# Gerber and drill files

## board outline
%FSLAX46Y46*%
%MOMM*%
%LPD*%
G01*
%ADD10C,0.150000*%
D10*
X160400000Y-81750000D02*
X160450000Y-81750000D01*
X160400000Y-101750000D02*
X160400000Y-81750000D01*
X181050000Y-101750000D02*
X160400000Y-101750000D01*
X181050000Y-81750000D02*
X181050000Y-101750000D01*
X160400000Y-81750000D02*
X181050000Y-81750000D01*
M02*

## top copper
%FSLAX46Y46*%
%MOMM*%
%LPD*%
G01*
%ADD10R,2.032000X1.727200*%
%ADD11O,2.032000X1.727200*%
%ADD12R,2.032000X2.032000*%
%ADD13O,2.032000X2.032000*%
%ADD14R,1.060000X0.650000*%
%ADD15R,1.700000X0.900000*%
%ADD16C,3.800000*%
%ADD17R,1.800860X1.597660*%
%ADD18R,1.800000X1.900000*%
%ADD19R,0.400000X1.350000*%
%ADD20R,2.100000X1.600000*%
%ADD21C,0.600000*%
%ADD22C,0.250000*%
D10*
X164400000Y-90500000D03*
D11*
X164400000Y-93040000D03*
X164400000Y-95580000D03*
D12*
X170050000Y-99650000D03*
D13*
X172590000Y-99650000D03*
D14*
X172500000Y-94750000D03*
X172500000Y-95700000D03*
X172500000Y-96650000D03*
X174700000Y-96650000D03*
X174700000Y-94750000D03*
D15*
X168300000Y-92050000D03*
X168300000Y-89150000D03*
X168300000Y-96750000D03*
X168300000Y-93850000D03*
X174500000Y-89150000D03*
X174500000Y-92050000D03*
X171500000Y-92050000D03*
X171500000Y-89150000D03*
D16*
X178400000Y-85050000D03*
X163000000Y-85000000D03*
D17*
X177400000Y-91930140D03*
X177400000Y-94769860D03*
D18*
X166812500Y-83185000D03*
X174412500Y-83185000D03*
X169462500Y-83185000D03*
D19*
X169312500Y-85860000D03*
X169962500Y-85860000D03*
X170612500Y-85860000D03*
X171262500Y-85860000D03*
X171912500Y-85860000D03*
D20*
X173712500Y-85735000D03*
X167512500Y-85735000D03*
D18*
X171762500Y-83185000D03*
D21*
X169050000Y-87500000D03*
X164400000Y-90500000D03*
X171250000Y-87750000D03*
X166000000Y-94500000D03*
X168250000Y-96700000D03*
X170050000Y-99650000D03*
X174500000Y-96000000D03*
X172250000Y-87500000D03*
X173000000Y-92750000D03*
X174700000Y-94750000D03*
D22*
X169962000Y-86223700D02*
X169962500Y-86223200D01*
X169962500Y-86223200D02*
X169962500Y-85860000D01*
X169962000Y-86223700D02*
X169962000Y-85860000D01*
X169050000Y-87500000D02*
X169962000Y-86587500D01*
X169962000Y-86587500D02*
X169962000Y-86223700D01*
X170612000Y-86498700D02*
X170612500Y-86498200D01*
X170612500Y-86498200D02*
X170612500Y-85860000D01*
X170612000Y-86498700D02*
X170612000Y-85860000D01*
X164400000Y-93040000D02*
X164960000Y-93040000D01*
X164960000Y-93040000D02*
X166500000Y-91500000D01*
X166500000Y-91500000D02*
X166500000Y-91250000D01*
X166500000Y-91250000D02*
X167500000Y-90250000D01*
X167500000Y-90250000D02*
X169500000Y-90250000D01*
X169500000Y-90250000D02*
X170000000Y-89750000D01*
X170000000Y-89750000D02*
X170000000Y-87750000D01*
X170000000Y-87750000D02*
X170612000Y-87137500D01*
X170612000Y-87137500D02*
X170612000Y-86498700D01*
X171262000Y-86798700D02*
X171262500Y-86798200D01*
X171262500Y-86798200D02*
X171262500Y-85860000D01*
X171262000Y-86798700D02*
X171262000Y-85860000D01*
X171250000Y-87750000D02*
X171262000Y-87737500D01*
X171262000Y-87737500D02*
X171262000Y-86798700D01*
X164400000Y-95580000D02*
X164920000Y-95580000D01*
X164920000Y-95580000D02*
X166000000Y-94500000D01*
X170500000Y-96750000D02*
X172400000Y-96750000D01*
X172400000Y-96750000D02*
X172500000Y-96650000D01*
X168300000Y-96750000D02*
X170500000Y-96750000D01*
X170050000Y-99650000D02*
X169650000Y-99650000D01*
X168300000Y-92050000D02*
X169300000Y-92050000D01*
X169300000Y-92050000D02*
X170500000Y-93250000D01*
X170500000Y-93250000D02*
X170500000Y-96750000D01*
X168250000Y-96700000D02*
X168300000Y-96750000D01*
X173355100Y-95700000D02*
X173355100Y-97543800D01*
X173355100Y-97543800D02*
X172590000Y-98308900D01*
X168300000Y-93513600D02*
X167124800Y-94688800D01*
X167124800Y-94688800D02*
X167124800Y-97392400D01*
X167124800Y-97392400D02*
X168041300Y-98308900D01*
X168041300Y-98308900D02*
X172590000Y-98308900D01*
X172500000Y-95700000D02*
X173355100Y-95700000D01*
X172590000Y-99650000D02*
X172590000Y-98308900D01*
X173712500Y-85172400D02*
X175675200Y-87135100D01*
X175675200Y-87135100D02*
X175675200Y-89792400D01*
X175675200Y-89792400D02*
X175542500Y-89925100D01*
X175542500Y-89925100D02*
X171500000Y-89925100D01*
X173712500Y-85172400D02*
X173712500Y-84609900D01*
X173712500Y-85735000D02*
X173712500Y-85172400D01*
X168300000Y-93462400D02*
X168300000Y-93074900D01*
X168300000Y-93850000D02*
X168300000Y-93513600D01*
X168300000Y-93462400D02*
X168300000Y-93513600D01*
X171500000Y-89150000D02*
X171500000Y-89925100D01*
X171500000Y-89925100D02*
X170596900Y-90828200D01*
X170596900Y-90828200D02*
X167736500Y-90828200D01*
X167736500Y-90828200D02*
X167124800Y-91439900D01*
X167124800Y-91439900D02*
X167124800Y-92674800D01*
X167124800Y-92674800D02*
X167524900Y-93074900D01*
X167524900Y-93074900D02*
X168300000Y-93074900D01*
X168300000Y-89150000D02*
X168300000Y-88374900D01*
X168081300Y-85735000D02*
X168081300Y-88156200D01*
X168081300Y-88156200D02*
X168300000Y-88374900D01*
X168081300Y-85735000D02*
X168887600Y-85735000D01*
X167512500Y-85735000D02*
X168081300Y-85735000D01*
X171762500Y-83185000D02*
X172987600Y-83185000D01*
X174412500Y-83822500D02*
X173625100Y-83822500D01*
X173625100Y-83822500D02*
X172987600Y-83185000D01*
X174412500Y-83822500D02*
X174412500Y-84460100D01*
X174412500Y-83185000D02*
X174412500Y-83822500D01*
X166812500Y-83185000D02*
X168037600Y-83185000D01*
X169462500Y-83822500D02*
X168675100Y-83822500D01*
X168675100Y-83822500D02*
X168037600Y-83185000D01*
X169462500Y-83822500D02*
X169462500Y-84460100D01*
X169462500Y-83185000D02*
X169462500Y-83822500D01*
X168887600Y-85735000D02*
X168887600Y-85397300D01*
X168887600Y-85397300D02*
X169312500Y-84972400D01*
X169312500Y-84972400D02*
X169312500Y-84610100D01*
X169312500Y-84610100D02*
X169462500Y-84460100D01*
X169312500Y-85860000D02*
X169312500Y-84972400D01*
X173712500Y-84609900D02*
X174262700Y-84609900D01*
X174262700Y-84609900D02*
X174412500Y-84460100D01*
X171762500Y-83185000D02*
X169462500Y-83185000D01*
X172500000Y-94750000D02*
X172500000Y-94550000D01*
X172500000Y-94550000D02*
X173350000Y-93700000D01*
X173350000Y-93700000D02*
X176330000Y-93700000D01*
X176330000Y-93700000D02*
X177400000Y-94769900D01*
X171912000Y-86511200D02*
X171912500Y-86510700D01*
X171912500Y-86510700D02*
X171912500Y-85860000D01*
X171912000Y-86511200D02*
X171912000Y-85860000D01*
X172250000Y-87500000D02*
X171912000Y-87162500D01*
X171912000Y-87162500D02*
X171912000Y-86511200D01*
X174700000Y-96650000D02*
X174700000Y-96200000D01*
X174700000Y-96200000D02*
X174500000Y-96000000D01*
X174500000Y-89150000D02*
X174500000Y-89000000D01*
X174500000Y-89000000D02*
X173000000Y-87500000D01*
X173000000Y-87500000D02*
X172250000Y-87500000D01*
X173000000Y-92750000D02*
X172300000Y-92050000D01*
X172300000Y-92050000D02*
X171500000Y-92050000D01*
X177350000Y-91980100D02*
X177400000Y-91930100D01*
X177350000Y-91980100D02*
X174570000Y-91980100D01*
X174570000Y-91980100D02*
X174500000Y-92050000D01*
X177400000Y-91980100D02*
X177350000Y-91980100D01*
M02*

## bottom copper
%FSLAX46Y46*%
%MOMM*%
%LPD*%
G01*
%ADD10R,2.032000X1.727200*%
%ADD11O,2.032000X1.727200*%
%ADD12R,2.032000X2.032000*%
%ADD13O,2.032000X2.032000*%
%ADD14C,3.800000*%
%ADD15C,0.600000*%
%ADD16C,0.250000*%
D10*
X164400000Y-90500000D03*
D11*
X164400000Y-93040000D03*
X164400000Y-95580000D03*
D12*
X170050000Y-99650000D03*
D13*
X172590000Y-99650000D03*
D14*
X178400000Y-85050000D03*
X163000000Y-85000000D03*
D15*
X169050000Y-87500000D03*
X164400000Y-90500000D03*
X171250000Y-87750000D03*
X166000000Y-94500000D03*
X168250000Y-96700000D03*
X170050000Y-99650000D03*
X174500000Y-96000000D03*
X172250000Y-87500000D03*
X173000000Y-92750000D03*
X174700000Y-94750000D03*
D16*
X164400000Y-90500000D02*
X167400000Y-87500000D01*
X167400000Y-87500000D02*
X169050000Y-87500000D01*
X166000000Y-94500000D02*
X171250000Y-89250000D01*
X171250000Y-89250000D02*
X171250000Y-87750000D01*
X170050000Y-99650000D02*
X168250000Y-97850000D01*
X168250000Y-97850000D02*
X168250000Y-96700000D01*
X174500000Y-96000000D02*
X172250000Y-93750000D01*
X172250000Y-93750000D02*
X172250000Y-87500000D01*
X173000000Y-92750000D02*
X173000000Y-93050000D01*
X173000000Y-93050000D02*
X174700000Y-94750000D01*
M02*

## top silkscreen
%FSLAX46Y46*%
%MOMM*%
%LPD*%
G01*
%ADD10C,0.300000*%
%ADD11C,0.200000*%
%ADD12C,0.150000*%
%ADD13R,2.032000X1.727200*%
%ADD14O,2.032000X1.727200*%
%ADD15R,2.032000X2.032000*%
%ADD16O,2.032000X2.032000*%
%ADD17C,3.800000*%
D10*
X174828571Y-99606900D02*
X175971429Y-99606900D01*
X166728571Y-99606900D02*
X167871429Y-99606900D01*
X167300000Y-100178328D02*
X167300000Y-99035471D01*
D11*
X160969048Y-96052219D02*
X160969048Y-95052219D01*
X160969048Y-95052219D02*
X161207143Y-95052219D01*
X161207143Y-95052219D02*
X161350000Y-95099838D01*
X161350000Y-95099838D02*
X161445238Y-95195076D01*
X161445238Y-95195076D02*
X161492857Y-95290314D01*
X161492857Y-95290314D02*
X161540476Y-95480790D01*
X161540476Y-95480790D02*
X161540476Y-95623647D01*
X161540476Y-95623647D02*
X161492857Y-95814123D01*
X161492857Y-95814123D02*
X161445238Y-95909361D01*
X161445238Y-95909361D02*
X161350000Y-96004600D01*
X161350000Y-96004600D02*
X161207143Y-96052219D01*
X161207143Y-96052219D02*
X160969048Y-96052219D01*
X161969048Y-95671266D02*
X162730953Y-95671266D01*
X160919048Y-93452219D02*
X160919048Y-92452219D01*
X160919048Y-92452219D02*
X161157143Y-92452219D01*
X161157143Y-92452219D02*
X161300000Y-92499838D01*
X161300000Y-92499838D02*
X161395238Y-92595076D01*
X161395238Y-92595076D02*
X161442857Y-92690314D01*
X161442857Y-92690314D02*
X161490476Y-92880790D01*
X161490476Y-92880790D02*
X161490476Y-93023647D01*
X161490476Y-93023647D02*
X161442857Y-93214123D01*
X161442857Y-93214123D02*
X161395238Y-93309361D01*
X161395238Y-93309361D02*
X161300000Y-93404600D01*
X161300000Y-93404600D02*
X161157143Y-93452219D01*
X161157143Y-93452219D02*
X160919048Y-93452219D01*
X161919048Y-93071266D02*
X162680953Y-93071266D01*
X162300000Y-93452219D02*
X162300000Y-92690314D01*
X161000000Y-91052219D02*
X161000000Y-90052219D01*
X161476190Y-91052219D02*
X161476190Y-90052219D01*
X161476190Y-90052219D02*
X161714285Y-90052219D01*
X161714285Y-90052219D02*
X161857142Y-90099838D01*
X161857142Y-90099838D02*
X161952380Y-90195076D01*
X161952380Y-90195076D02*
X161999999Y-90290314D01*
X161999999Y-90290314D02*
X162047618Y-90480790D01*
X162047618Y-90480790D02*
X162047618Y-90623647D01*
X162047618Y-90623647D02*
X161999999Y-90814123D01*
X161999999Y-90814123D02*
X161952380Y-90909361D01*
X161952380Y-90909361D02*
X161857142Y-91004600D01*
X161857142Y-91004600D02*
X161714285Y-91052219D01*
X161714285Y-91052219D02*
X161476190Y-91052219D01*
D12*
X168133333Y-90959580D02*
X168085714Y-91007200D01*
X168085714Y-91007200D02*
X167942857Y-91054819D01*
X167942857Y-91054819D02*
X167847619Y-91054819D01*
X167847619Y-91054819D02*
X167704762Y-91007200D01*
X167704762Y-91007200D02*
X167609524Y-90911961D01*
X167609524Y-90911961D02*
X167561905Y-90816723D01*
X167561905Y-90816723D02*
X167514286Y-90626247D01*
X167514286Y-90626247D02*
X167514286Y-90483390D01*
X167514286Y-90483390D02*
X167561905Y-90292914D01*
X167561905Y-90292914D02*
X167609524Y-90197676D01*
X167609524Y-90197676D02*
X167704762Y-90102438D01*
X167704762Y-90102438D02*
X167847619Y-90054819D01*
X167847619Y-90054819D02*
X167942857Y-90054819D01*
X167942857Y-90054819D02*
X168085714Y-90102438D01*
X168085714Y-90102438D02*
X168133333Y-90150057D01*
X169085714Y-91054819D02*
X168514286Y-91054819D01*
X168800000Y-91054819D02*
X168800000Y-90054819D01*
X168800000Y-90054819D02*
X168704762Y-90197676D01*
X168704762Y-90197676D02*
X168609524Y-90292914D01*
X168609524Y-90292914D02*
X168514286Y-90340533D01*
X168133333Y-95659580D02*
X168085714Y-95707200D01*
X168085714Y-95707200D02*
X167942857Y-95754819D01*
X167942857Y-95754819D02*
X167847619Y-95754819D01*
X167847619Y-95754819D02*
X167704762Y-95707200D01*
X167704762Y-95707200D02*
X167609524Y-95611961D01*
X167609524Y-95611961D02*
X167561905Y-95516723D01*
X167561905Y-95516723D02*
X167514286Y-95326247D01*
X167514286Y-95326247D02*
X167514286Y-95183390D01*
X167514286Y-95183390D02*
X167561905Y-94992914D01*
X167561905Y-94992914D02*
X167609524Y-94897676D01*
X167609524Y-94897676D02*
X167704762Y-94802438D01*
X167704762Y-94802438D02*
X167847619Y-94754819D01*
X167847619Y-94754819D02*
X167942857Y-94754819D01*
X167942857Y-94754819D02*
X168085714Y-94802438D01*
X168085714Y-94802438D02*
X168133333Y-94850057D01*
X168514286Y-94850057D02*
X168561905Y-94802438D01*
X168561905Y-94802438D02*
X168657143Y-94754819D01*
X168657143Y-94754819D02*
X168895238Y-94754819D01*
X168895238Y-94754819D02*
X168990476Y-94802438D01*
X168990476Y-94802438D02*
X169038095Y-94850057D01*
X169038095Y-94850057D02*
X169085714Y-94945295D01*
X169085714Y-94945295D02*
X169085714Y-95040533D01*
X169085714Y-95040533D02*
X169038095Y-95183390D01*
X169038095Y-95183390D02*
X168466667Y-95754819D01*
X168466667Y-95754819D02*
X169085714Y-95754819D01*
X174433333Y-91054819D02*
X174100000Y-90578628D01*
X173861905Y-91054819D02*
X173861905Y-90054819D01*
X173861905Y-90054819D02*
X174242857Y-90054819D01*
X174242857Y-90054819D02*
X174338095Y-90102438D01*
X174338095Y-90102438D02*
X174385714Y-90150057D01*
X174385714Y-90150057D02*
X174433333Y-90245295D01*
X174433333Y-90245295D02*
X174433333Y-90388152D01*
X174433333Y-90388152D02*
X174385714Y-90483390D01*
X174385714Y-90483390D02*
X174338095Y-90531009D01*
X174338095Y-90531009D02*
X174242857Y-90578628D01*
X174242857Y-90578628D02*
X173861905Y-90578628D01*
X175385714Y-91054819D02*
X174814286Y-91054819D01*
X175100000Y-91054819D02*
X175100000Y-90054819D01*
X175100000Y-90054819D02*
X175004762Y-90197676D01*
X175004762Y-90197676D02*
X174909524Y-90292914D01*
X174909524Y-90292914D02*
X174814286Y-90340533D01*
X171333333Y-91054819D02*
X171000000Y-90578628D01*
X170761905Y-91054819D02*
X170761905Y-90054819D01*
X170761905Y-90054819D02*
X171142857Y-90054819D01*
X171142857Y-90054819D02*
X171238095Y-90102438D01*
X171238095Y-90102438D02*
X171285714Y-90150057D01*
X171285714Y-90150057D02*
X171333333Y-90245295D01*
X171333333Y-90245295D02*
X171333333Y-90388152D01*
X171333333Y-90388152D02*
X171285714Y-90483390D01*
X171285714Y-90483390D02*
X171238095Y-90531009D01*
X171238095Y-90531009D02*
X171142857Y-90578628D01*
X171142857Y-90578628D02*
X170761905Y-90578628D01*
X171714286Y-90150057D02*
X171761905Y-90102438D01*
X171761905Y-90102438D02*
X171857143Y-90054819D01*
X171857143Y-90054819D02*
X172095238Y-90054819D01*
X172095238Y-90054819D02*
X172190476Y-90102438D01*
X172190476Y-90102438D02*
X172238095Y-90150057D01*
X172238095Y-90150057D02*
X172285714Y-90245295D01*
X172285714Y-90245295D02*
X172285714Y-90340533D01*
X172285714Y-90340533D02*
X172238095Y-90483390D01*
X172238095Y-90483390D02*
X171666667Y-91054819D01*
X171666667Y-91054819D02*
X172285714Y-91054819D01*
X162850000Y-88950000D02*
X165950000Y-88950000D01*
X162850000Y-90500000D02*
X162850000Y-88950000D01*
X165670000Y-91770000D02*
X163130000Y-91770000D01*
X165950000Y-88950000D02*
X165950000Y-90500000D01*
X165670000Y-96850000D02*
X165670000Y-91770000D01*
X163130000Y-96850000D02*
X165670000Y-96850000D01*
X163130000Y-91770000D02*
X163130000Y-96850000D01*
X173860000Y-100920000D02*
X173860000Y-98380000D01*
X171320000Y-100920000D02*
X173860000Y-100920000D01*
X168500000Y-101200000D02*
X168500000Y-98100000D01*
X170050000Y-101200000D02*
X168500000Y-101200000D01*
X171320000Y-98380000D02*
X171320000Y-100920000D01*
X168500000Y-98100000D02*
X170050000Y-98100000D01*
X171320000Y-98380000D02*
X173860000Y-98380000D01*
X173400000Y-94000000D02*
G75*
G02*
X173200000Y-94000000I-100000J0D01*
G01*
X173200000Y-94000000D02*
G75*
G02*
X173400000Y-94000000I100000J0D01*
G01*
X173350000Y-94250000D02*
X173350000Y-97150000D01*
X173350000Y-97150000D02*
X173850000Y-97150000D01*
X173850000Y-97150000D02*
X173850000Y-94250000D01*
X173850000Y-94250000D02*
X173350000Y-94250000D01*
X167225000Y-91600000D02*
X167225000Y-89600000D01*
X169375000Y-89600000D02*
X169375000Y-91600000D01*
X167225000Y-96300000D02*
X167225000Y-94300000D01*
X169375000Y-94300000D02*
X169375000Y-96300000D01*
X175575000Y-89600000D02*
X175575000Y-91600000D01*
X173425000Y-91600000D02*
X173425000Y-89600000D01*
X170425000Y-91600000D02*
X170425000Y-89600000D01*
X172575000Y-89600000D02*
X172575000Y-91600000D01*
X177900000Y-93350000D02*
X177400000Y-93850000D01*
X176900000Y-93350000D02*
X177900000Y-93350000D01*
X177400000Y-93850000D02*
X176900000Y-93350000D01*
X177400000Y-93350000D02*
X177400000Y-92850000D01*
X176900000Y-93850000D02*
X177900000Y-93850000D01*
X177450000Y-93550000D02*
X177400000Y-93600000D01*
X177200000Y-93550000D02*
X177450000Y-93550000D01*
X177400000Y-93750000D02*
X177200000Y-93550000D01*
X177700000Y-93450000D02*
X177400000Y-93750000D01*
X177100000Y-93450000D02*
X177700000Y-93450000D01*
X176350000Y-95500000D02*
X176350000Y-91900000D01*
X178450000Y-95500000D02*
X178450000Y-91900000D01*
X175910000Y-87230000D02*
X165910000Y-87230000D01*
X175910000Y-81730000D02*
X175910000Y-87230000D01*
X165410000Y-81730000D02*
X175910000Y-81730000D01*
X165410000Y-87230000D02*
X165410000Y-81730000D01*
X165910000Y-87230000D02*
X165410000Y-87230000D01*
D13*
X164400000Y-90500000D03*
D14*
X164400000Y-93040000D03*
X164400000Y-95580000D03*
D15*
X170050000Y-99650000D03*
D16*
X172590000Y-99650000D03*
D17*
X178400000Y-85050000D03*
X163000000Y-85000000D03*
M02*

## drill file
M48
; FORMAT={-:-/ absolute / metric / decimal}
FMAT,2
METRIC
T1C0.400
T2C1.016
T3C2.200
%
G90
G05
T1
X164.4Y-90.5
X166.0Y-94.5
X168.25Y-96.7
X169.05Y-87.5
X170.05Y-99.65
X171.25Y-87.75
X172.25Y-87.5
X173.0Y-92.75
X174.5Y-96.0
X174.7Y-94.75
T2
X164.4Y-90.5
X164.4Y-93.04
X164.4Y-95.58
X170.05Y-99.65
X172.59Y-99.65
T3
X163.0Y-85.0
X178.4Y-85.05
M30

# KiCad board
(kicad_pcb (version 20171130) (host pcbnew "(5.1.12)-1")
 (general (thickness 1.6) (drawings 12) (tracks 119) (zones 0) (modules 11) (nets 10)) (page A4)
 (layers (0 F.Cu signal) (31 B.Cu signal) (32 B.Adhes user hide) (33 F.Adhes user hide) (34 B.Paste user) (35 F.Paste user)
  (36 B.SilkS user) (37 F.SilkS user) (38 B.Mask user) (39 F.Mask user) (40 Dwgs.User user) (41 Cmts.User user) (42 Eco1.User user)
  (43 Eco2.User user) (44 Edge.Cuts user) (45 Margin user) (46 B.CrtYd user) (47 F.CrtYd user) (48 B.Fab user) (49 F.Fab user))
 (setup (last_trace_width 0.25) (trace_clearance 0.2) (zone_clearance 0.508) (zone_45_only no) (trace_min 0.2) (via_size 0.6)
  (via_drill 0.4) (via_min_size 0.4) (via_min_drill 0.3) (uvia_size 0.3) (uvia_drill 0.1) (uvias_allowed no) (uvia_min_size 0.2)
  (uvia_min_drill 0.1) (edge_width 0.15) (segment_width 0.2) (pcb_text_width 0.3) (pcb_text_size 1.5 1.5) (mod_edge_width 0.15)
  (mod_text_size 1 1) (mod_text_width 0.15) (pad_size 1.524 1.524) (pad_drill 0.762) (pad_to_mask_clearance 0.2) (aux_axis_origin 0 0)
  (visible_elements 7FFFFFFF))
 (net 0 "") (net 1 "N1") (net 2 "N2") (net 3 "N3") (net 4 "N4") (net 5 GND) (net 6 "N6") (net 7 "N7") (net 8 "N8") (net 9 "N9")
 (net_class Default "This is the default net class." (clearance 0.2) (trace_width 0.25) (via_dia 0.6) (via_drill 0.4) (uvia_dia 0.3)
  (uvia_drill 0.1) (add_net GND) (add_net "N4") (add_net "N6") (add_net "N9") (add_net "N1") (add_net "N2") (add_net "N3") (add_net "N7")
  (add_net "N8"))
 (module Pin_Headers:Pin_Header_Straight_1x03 (layer F.Cu) (at 164.4 90.5)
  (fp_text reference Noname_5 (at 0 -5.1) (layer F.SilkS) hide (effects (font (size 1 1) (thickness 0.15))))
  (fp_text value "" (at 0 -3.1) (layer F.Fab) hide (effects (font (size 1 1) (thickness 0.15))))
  (fp_line (start -1.55 -1.55) (end 1.55 -1.55) (layer F.SilkS) (width 0.15))
  (fp_line (start -1.55 0) (end -1.55 -1.55) (layer F.SilkS) (width 0.15))
  (fp_line (start 1.27 1.27) (end -1.27 1.27) (layer F.SilkS) (width 0.15))
  (fp_line (start 1.55 -1.55) (end 1.55 0) (layer F.SilkS) (width 0.15))
  (fp_line (start 1.27 6.35) (end 1.27 1.27) (layer F.SilkS) (width 0.15))
  (fp_line (start -1.27 6.35) (end 1.27 6.35) (layer F.SilkS) (width 0.15))
  (fp_line (start -1.27 1.27) (end -1.27 6.35) (layer F.SilkS) (width 0.15))
  (pad 1 thru_hole rect (at 0 0) (size 2.032 1.7272) (drill 1.016) (layers *.Cu *.Mask F.SilkS) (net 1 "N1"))
  (pad 2 thru_hole oval (at 0 2.54) (size 2.032 1.7272) (drill 1.016) (layers *.Cu *.Mask F.SilkS) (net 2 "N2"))
  (pad 3 thru_hole oval (at 0 5.08) (size 2.032 1.7272) (drill 1.016) (layers *.Cu *.Mask F.SilkS) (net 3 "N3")))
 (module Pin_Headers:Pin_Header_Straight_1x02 (layer F.Cu) (at 170.05 99.65 90)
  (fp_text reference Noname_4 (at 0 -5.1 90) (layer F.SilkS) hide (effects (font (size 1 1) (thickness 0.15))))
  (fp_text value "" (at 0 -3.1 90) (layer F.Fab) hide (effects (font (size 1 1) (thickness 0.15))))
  (fp_line (start -1.27 3.81) (end 1.27 3.81) (layer F.SilkS) (width 0.15))
  (fp_line (start -1.27 1.27) (end -1.27 3.81) (layer F.SilkS) (width 0.15))
  (fp_line (start -1.55 -1.55) (end 1.55 -1.55) (layer F.SilkS) (width 0.15))
  (fp_line (start -1.55 0) (end -1.55 -1.55) (layer F.SilkS) (width 0.15))
  (fp_line (start 1.27 1.27) (end -1.27 1.27) (layer F.SilkS) (width 0.15))
  (fp_line (start 1.55 -1.55) (end 1.55 0) (layer F.SilkS) (width 0.15))
  (fp_line (start 1.27 1.27) (end 1.27 3.81) (layer F.SilkS) (width 0.15))
  (pad 1 thru_hole rect (at 0 0 90) (size 2.032 2.032) (drill 1.016) (layers *.Cu *.Mask F.SilkS) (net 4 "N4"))
  (pad 2 thru_hole oval (at 0 2.54 90) (size 2.032 2.032) (drill 1.016) (layers *.Cu *.Mask F.SilkS) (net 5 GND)))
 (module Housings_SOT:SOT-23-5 (layer F.Cu) (at 173.6 95.7) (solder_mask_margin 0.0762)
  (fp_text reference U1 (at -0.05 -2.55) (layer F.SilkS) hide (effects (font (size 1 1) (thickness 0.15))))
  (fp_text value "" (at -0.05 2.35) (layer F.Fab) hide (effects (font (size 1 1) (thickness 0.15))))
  (fp_circle (center -0.3 -1.7) (end -0.2 -1.7) (layer F.SilkS) (width 0.15))
  (fp_line (start -0.25 -1.45) (end -0.25 1.45) (layer F.SilkS) (width 0.15))
  (fp_line (start -0.25 1.45) (end 0.25 1.45) (layer F.SilkS) (width 0.15))
  (fp_line (start 0.25 1.45) (end 0.25 -1.45) (layer F.SilkS) (width 0.15))
  (fp_line (start 0.25 -1.45) (end -0.25 -1.45) (layer F.SilkS) (width 0.15))
  (pad 1 smd rect (at -1.1 -0.95) (size 1.06 0.65) (layers F.Cu F.Paste F.Mask) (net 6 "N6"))
  (pad 2 smd rect (at -1.1 0) (size 1.06 0.65) (layers F.Cu F.Paste F.Mask) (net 5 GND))
  (pad 3 smd rect (at -1.1 0.95) (size 1.06 0.65) (layers F.Cu F.Paste F.Mask) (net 4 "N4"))
  (pad 4 smd rect (at 1.1 0.95) (size 1.06 0.65) (layers F.Cu F.Paste F.Mask) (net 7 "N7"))
  (pad 5 smd rect (at 1.1 -0.95) (size 1.06 0.65) (layers F.Cu F.Paste F.Mask) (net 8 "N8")))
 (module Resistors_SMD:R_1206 (layer F.Cu) (at 168.3 90.6 90)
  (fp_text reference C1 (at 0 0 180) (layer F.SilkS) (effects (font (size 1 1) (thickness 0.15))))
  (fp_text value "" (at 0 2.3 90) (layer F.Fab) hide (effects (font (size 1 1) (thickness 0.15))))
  (fp_line (start -1 -1.075) (end 1 -1.075) (layer F.SilkS) (width 0.15))
  (fp_line (start 1 1.075) (end -1 1.075) (layer F.SilkS) (width 0.15))
  (pad 1 smd rect (at -1.45 0 90) (size 0.9 1.7) (layers F.Cu F.Paste F.Mask) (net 4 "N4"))
  (pad 2 smd rect (at 1.45 0 90) (size 0.9 1.7) (layers F.Cu F.Paste F.Mask) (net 5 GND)))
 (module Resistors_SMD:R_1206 (layer F.Cu) (at 168.3 95.3 90)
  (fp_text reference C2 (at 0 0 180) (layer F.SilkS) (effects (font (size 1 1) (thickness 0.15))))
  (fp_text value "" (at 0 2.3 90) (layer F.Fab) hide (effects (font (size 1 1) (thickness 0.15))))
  (fp_line (start -1 -1.075) (end 1 -1.075) (layer F.SilkS) (width 0.15))
  (fp_line (start 1 1.075) (end -1 1.075) (layer F.SilkS) (width 0.15))
  (pad 1 smd rect (at -1.45 0 90) (size 0.9 1.7) (layers F.Cu F.Paste F.Mask) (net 4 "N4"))
  (pad 2 smd rect (at 1.45 0 90) (size 0.9 1.7) (layers F.Cu F.Paste F.Mask) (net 5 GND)))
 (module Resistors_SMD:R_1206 (layer F.Cu) (at 174.5 90.6 270)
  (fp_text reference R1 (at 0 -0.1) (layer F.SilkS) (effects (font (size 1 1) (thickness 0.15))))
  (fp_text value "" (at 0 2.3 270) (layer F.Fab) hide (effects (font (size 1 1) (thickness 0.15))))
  (fp_line (start -1 -1.075) (end 1 -1.075) (layer F.SilkS) (width 0.15))
  (fp_line (start 1 1.075) (end -1 1.075) (layer F.SilkS) (width 0.15))
  (pad 1 smd rect (at -1.45 0 270) (size 0.9 1.7) (layers F.Cu F.Paste F.Mask) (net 7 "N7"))
  (pad 2 smd rect (at 1.45 0 270) (size 0.9 1.7) (layers F.Cu F.Paste F.Mask) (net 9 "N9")))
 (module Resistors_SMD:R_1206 (layer F.Cu) (at 171.5 90.6 90)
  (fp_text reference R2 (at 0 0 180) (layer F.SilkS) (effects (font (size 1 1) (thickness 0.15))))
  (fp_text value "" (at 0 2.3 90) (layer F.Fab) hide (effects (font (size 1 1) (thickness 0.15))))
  (fp_line (start -1 -1.075) (end 1 -1.075) (layer F.SilkS) (width 0.15))
  (fp_line (start 1 1.075) (end -1 1.075) (layer F.SilkS) (width 0.15))
  (pad 1 smd rect (at -1.45 0 90) (size 0.9 1.7) (layers F.Cu F.Paste F.Mask) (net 8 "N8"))
  (pad 2 smd rect (at 1.45 0 90) (size 0.9 1.7) (layers F.Cu F.Paste F.Mask) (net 5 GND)))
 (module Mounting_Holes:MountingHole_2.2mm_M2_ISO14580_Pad (layer F.Cu) (at 178.4 85.05)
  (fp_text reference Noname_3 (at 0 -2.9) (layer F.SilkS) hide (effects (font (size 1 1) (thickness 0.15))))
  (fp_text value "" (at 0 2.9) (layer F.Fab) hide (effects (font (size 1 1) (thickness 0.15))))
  (pad 1 thru_hole circle (at 0 0) (size 3.8 3.8) (drill 2.2) (layers *.Cu *.Mask F.SilkS)))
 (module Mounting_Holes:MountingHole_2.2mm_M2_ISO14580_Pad (layer F.Cu) (at 163 85)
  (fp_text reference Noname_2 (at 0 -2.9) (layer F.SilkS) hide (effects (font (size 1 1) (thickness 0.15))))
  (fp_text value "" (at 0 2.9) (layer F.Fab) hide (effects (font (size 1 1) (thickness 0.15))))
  (pad 1 thru_hole circle (at 0 0) (size 3.8 3.8) (drill 2.2) (layers *.Cu *.Mask F.SilkS)))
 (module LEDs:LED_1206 (layer F.Cu) (at 177.4 93.35 90)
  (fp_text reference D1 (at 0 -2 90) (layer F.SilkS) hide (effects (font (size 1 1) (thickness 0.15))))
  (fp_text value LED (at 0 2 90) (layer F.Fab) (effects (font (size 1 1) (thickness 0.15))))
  (fp_line (start 0 0.5) (end -0.5 0) (layer F.SilkS) (width 0.15))
  (fp_line (start 0 -0.5) (end 0 0.5) (layer F.SilkS) (width 0.15))
  (fp_line (start -0.5 0) (end 0 -0.5) (layer F.SilkS) (width 0.15))
  (fp_line (start 0 0) (end 0.5 0) (layer F.SilkS) (width 0.15))
  (fp_line (start -0.5 -0.5) (end -0.5 0.5) (layer F.SilkS) (width 0.15))
  (fp_line (start -0.2 0.05) (end -0.25 0) (layer F.SilkS) (width 0.15))
  (fp_line (start -0.2 -0.2) (end -0.2 0.05) (layer F.SilkS) (width 0.15))
  (fp_line (start -0.4 0) (end -0.2 -0.2) (layer F.SilkS) (width 0.15))
  (fp_line (start -0.1 0.3) (end -0.4 0) (layer F.SilkS) (width 0.15))
  (fp_line (start -0.1 -0.3) (end -0.1 0.3) (layer F.SilkS) (width 0.15))
  (fp_line (start -2.15 -1.05) (end 1.45 -1.05) (layer F.SilkS) (width 0.15))
  (fp_line (start -2.15 1.05) (end 1.45 1.05) (layer F.SilkS) (width 0.15))
  (pad 2 smd rect (at 1.41986 0 270) (size 1.59766 1.80086) (layers F.Cu F.Paste F.Mask) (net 9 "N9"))
  (pad 1 smd rect (at -1.41986 0 270) (size 1.59766 1.80086) (layers F.Cu F.Paste F.Mask) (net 6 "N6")))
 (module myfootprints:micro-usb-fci (layer F.Cu) (at 171.2 84.2) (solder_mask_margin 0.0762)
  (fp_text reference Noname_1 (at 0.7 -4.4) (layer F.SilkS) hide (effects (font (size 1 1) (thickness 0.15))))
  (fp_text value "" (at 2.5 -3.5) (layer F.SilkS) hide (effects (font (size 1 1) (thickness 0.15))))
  (fp_line (start 4.71 3.03) (end -5.29 3.03) (layer F.SilkS) (width 0.15))
  (fp_line (start 4.71 -2.47) (end 4.71 3.03) (layer F.SilkS) (width 0.15))
  (fp_line (start -5.79 -2.47) (end 4.71 -2.47) (layer F.SilkS) (width 0.15))
  (fp_line (start -5.79 3.03) (end -5.79 -2.47) (layer F.SilkS) (width 0.15))
  (fp_line (start -5.29 3.03) (end -5.79 3.03) (layer F.SilkS) (width 0.15))
  (pad 6 smd rect (at -4.3875 -1.015) (size 1.8 1.9) (layers F.Cu F.Paste F.Mask) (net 5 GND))
  (pad 6 smd rect (at 3.2125 -1.015) (size 1.8 1.9) (layers F.Cu F.Paste F.Mask) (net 5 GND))
  (pad 6 smd rect (at -1.7375 -1.015) (size 1.8 1.9) (layers F.Cu F.Paste F.Mask) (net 5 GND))
  (pad 5 smd rect (at -1.8875 1.66) (size 0.4 1.35) (layers F.Cu F.Paste F.Mask) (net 5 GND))
  (pad 4 smd rect (at -1.2375 1.66) (size 0.4 1.35) (layers F.Cu F.Paste F.Mask) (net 1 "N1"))
  (pad 3 smd rect (at -0.5875 1.66) (size 0.4 1.35) (layers F.Cu F.Paste F.Mask) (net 2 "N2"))
  (pad 2 smd rect (at 0.0625 1.66) (size 0.4 1.35) (layers F.Cu F.Paste F.Mask) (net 3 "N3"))
  (pad 1 smd rect (at 0.7125 1.66) (size 0.4 1.35) (layers F.Cu F.Paste F.Mask) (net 7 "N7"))
  (pad 6 smd rect (at 2.5125 1.535) (size 2.1 1.6) (layers F.Cu F.Paste F.Mask) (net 5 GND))
  (pad 6 smd rect (at -3.6875 1.535) (size 2.1 1.6) (layers F.Cu F.Paste F.Mask) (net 5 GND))
  (pad 6 smd rect (at 0.5625 -1.015) (size 1.8 1.9) (layers F.Cu F.Paste F.Mask) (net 5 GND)))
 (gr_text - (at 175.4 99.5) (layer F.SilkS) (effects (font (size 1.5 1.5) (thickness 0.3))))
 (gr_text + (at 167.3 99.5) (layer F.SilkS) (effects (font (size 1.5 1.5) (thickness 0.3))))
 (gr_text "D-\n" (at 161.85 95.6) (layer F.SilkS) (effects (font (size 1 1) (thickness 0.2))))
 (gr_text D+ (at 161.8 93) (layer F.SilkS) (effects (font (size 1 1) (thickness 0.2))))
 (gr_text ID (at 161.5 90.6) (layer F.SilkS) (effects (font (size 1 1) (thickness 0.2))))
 (gr_line (start 160.4 81.75) (end 160.45 81.75) (angle 90) (layer Edge.Cuts) (width 0.15))
 (gr_line (start 160.4 101.75) (end 160.4 81.75) (angle 90) (layer Edge.Cuts) (width 0.15))
 (gr_line (start 181.05 101.75) (end 160.4 101.75) (angle 90) (layer Edge.Cuts) (width 0.15))
 (gr_line (start 181.05 81.75) (end 181.05 101.75) (angle 90) (layer Edge.Cuts) (width 0.15))
 (gr_line (start 160.4 81.75) (end 181.05 81.75) (angle 90) (layer Edge.Cuts) (width 0.15))
 (segment (start 169.962 86.2237) (end 169.9625 86.2232) (width 0.25) (layer F.Cu) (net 1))
 (segment (start 169.9625 86.2232) (end 169.9625 85.86) (width 0.25) (layer F.Cu) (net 1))
 (segment (start 169.962 86.2237) (end 169.962 85.86) (width 0.25) (layer F.Cu) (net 1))
 (segment (start 169.05 87.5) (end 169.962 86.5875) (width 0.25) (layer F.Cu) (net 1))
 (segment (start 169.962 86.5875) (end 169.962 86.2237) (width 0.25) (layer F.Cu) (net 1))
 (segment (start 164.4 90.5) (end 167.4 87.5) (width 0.25) (layer B.Cu) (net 1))
 (segment (start 167.4 87.5) (end 169.05 87.5) (width 0.25) (layer B.Cu) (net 1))
 (via (at 169.05 87.5) (size 0.6) (layers F.Cu B.Cu) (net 1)) (via (at 164.4 90.5) (size 0.6) (layers F.Cu B.Cu) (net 1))
 (segment (start 170.612 86.4987) (end 170.6125 86.4982) (width 0.25) (layer F.Cu) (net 2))
 (segment (start 170.6125 86.4982) (end 170.6125 85.86) (width 0.25) (layer F.Cu) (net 2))
 (segment (start 170.612 86.4987) (end 170.612 85.86) (width 0.25) (layer F.Cu) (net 2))
 (segment (start 164.4 93.04) (end 164.96 93.04) (width 0.25) (layer F.Cu) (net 2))
 (segment (start 164.96 93.04) (end 166.5 91.5) (width 0.25) (layer F.Cu) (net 2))
 (segment (start 166.5 91.5) (end 166.5 91.25) (width 0.25) (layer F.Cu) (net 2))
 (segment (start 166.5 91.25) (end 167.5 90.25) (width 0.25) (layer F.Cu) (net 2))
 (segment (start 167.5 90.25) (end 169.5 90.25) (width 0.25) (layer F.Cu) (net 2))
 (segment (start 169.5 90.25) (end 170 89.75) (width 0.25) (layer F.Cu) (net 2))
 (segment (start 170 89.75) (end 170 87.75) (width 0.25) (layer F.Cu) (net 2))
 (segment (start 170 87.75) (end 170.612 87.1375) (width 0.25) (layer F.Cu) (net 2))
 (segment (start 170.612 87.1375) (end 170.612 86.4987) (width 0.25) (layer F.Cu) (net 2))
 (segment (start 171.262 86.7987) (end 171.2625 86.7982) (width 0.25) (layer F.Cu) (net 3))
 (segment (start 171.2625 86.7982) (end 171.2625 85.86) (width 0.25) (layer F.Cu) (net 3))
 (segment (start 171.262 86.7987) (end 171.262 85.86) (width 0.25) (layer F.Cu) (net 3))
 (segment (start 171.25 87.75) (end 171.262 87.7375) (width 0.25) (layer F.Cu) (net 3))
 (segment (start 171.262 87.7375) (end 171.262 86.7987) (width 0.25) (layer F.Cu) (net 3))
 (segment (start 166 94.5) (end 171.25 89.25) (width 0.25) (layer B.Cu) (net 3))
 (segment (start 171.25 89.25) (end 171.25 87.75) (width 0.25) (layer B.Cu) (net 3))
 (segment (start 164.4 95.58) (end 164.92 95.58) (width 0.25) (layer F.Cu) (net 3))
 (segment (start 164.92 95.58) (end 166 94.5) (width 0.25) (layer F.Cu) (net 3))
 (via (at 171.25 87.75) (size 0.6) (layers F.Cu B.Cu) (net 3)) (via (at 166 94.5) (size 0.6) (layers F.Cu B.Cu) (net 3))
 (segment (start 170.5 96.75) (end 172.4 96.75) (width 0.25) (layer F.Cu) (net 4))
 (segment (start 172.4 96.75) (end 172.5 96.65) (width 0.25) (layer F.Cu) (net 4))
 (segment (start 168.3 96.75) (end 170.5 96.75) (width 0.25) (layer F.Cu) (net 4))
 (segment (start 170.05 99.65) (end 169.65 99.65) (width 0.25) (layer F.Cu) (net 4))
 (segment (start 168.3 92.05) (end 169.3 92.05) (width 0.25) (layer F.Cu) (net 4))
 (segment (start 169.3 92.05) (end 170.5 93.25) (width 0.25) (layer F.Cu) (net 4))
 (segment (start 170.5 93.25) (end 170.5 96.75) (width 0.25) (layer F.Cu) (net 4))
 (segment (start 170.05 99.65) (end 168.25 97.85) (width 0.25) (layer B.Cu) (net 4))
 (segment (start 168.25 97.85) (end 168.25 96.7) (width 0.25) (layer B.Cu) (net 4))
 (segment (start 168.25 96.7) (end 168.3 96.75) (width 0.25) (layer F.Cu) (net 4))
 (via (at 168.25 96.7) (size 0.6) (layers F.Cu B.Cu) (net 4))
 (via (at 170.05 99.65) (size 0.6) (layers F.Cu B.Cu) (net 4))
 (segment (start 173.3551 95.7) (end 173.3551 97.5438) (width 0.25) (layer F.Cu) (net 5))
 (segment (start 173.3551 97.5438) (end 172.59 98.3089) (width 0.25) (layer F.Cu) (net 5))
 (segment (start 168.3 93.5136) (end 167.1248 94.6888) (width 0.25) (layer F.Cu) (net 5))
 (segment (start 167.1248 94.6888) (end 167.1248 97.3924) (width 0.25) (layer F.Cu) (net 5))
 (segment (start 167.1248 97.3924) (end 168.0413 98.3089) (width 0.25) (layer F.Cu) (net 5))
 (segment (start 168.0413 98.3089) (end 172.59 98.3089) (width 0.25) (layer F.Cu) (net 5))
 (segment (start 172.5 95.7) (end 173.3551 95.7) (width 0.25) (layer F.Cu) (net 5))
 (segment (start 172.59 99.65) (end 172.59 98.3089) (width 0.25) (layer F.Cu) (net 5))
 (segment (start 173.7125 85.1724) (end 175.6752 87.1351) (width 0.25) (layer F.Cu) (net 5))
 (segment (start 175.6752 87.1351) (end 175.6752 89.7924) (width 0.25) (layer F.Cu) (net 5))
 (segment (start 175.6752 89.7924) (end 175.5425 89.9251) (width 0.25) (layer F.Cu) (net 5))
 (segment (start 175.5425 89.9251) (end 171.5 89.9251) (width 0.25) (layer F.Cu) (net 5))
 (segment (start 173.7125 85.1724) (end 173.7125 84.6099) (width 0.25) (layer F.Cu) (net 5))
 (segment (start 173.7125 85.735) (end 173.7125 85.1724) (width 0.25) (layer F.Cu) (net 5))
 (segment (start 168.3 93.4624) (end 168.3 93.0749) (width 0.25) (layer F.Cu) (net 5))
 (segment (start 168.3 93.85) (end 168.3 93.5136) (width 0.25) (layer F.Cu) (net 5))
 (segment (start 168.3 93.4624) (end 168.3 93.5136) (width 0.25) (layer F.Cu) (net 5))
 (segment (start 171.5 89.15) (end 171.5 89.9251) (width 0.25) (layer F.Cu) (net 5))
 (segment (start 171.5 89.9251) (end 170.5969 90.8282) (width 0.25) (layer F.Cu) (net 5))
 (segment (start 170.5969 90.8282) (end 167.7365 90.8282) (width 0.25) (layer F.Cu) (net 5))
 (segment (start 167.7365 90.8282) (end 167.1248 91.4399) (width 0.25) (layer F.Cu) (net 5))
 (segment (start 167.1248 91.4399) (end 167.1248 92.6748) (width 0.25) (layer F.Cu) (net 5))
 (segment (start 167.1248 92.6748) (end 167.5249 93.0749) (width 0.25) (layer F.Cu) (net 5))
 (segment (start 167.5249 93.0749) (end 168.3 93.0749) (width 0.25) (layer F.Cu) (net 5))
 (segment (start 168.3 89.15) (end 168.3 88.3749) (width 0.25) (layer F.Cu) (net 5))
 (segment (start 168.0813 85.735) (end 168.0813 88.1562) (width 0.25) (layer F.Cu) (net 5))
 (segment (start 168.0813 88.1562) (end 168.3 88.3749) (width 0.25) (layer F.Cu) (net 5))
 (segment (start 168.0813 85.735) (end 168.8876 85.735) (width 0.25) (layer F.Cu) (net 5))
 (segment (start 167.5125 85.735) (end 168.0813 85.735) (width 0.25) (layer F.Cu) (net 5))
 (segment (start 171.7625 83.185) (end 172.9876 83.185) (width 0.25) (layer F.Cu) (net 5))
 (segment (start 174.4125 83.8225) (end 173.6251 83.8225) (width 0.25) (layer F.Cu) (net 5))
 (segment (start 173.6251 83.8225) (end 172.9876 83.185) (width 0.25) (layer F.Cu) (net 5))
 (segment (start 174.4125 83.8225) (end 174.4125 84.4601) (width 0.25) (layer F.Cu) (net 5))
 (segment (start 174.4125 83.185) (end 174.4125 83.8225) (width 0.25) (layer F.Cu) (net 5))
 (segment (start 166.8125 83.185) (end 168.0376 83.185) (width 0.25) (layer F.Cu) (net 5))
 (segment (start 169.4625 83.8225) (end 168.6751 83.8225) (width 0.25) (layer F.Cu) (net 5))
 (segment (start 168.6751 83.8225) (end 168.0376 83.185) (width 0.25) (layer F.Cu) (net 5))
 (segment (start 169.4625 83.8225) (end 169.4625 84.4601) (width 0.25) (layer F.Cu) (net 5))
 (segment (start 169.4625 83.185) (end 169.4625 83.8225) (width 0.25) (layer F.Cu) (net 5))
 (segment (start 168.8876 85.735) (end 168.8876 85.3973) (width 0.25) (layer F.Cu) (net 5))
 (segment (start 168.8876 85.3973) (end 169.3125 84.9724) (width 0.25) (layer F.Cu) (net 5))
 (segment (start 169.3125 84.9724) (end 169.3125 84.6101) (width 0.25) (layer F.Cu) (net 5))
 (segment (start 169.3125 84.6101) (end 169.4625 84.4601) (width 0.25) (layer F.Cu) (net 5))
 (segment (start 169.3125 85.86) (end 169.3125 84.9724) (width 0.25) (layer F.Cu) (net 5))
 (segment (start 173.7125 84.6099) (end 174.2627 84.6099) (width 0.25) (layer F.Cu) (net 5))
 (segment (start 174.2627 84.6099) (end 174.4125 84.4601) (width 0.25) (layer F.Cu) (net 5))
 (segment (start 171.7625 83.185) (end 169.4625 83.185) (width 0.25) (layer F.Cu) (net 5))
 (segment (start 172.5 94.75) (end 172.5 94.55) (width 0.25) (layer F.Cu) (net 6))
 (segment (start 172.5 94.55) (end 173.35 93.7) (width 0.25) (layer F.Cu) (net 6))
 (segment (start 173.35 93.7) (end 176.33 93.7) (width 0.25) (layer F.Cu) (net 6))
 (segment (start 176.33 93.7) (end 177.4 94.7699) (width 0.25) (layer F.Cu) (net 6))
 (segment (start 171.912 86.5112) (end 171.9125 86.5107) (width 0.25) (layer F.Cu) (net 7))
 (segment (start 171.9125 86.5107) (end 171.9125 85.86) (width 0.25) (layer F.Cu) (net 7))
 (segment (start 171.912 86.5112) (end 171.912 85.86) (width 0.25) (layer F.Cu) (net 7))
 (segment (start 172.25 87.5) (end 171.912 87.1625) (width 0.25) (layer F.Cu) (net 7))
 (segment (start 171.912 87.1625) (end 171.912 86.5112) (width 0.25) (layer F.Cu) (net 7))
 (segment (start 174.7 96.65) (end 174.7 96.2) (width 0.25) (layer F.Cu) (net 7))
 (segment (start 174.7 96.2) (end 174.5 96) (width 0.25) (layer F.Cu) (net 7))
 (segment (start 174.5 96) (end 172.25 93.75) (width 0.25) (layer B.Cu) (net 7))
 (segment (start 172.25 93.75) (end 172.25 87.5) (width 0.25) (layer B.Cu) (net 7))
 (segment (start 174.5 89.15) (end 174.5 89) (width 0.25) (layer F.Cu) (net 7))
 (segment (start 174.5 89) (end 173 87.5) (width 0.25) (layer F.Cu) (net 7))
 (segment (start 173 87.5) (end 172.25 87.5) (width 0.25) (layer F.Cu) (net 7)) (via (at 174.5 96) (size 0.6) (layers F.Cu B.Cu) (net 7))
 (via (at 172.25 87.5) (size 0.6) (layers F.Cu B.Cu) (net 7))
 (segment (start 173 92.75) (end 172.3 92.05) (width 0.25) (layer F.Cu) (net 8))
 (segment (start 172.3 92.05) (end 171.5 92.05) (width 0.25) (layer F.Cu) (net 8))
 (segment (start 173 92.75) (end 173 93.05) (width 0.25) (layer B.Cu) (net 8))
 (segment (start 173 93.05) (end 174.7 94.75) (width 0.25) (layer B.Cu) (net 8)) (via (at 173 92.75) (size 0.6) (layers F.Cu B.Cu) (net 8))
 (via (at 174.7 94.75) (size 0.6) (layers F.Cu B.Cu) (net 8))
 (segment (start 177.35 91.9801) (end 177.4 91.9301) (width 0.25) (layer F.Cu) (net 9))
 (segment (start 177.35 91.9801) (end 174.57 91.9801) (width 0.25) (layer F.Cu) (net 9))
 (segment (start 174.57 91.9801) (end 174.5 92.05) (width 0.25) (layer F.Cu) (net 9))
 (segment (start 177.4 91.9801) (end 177.35 91.9801) (width 0.25) (layer F.Cu) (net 9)))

